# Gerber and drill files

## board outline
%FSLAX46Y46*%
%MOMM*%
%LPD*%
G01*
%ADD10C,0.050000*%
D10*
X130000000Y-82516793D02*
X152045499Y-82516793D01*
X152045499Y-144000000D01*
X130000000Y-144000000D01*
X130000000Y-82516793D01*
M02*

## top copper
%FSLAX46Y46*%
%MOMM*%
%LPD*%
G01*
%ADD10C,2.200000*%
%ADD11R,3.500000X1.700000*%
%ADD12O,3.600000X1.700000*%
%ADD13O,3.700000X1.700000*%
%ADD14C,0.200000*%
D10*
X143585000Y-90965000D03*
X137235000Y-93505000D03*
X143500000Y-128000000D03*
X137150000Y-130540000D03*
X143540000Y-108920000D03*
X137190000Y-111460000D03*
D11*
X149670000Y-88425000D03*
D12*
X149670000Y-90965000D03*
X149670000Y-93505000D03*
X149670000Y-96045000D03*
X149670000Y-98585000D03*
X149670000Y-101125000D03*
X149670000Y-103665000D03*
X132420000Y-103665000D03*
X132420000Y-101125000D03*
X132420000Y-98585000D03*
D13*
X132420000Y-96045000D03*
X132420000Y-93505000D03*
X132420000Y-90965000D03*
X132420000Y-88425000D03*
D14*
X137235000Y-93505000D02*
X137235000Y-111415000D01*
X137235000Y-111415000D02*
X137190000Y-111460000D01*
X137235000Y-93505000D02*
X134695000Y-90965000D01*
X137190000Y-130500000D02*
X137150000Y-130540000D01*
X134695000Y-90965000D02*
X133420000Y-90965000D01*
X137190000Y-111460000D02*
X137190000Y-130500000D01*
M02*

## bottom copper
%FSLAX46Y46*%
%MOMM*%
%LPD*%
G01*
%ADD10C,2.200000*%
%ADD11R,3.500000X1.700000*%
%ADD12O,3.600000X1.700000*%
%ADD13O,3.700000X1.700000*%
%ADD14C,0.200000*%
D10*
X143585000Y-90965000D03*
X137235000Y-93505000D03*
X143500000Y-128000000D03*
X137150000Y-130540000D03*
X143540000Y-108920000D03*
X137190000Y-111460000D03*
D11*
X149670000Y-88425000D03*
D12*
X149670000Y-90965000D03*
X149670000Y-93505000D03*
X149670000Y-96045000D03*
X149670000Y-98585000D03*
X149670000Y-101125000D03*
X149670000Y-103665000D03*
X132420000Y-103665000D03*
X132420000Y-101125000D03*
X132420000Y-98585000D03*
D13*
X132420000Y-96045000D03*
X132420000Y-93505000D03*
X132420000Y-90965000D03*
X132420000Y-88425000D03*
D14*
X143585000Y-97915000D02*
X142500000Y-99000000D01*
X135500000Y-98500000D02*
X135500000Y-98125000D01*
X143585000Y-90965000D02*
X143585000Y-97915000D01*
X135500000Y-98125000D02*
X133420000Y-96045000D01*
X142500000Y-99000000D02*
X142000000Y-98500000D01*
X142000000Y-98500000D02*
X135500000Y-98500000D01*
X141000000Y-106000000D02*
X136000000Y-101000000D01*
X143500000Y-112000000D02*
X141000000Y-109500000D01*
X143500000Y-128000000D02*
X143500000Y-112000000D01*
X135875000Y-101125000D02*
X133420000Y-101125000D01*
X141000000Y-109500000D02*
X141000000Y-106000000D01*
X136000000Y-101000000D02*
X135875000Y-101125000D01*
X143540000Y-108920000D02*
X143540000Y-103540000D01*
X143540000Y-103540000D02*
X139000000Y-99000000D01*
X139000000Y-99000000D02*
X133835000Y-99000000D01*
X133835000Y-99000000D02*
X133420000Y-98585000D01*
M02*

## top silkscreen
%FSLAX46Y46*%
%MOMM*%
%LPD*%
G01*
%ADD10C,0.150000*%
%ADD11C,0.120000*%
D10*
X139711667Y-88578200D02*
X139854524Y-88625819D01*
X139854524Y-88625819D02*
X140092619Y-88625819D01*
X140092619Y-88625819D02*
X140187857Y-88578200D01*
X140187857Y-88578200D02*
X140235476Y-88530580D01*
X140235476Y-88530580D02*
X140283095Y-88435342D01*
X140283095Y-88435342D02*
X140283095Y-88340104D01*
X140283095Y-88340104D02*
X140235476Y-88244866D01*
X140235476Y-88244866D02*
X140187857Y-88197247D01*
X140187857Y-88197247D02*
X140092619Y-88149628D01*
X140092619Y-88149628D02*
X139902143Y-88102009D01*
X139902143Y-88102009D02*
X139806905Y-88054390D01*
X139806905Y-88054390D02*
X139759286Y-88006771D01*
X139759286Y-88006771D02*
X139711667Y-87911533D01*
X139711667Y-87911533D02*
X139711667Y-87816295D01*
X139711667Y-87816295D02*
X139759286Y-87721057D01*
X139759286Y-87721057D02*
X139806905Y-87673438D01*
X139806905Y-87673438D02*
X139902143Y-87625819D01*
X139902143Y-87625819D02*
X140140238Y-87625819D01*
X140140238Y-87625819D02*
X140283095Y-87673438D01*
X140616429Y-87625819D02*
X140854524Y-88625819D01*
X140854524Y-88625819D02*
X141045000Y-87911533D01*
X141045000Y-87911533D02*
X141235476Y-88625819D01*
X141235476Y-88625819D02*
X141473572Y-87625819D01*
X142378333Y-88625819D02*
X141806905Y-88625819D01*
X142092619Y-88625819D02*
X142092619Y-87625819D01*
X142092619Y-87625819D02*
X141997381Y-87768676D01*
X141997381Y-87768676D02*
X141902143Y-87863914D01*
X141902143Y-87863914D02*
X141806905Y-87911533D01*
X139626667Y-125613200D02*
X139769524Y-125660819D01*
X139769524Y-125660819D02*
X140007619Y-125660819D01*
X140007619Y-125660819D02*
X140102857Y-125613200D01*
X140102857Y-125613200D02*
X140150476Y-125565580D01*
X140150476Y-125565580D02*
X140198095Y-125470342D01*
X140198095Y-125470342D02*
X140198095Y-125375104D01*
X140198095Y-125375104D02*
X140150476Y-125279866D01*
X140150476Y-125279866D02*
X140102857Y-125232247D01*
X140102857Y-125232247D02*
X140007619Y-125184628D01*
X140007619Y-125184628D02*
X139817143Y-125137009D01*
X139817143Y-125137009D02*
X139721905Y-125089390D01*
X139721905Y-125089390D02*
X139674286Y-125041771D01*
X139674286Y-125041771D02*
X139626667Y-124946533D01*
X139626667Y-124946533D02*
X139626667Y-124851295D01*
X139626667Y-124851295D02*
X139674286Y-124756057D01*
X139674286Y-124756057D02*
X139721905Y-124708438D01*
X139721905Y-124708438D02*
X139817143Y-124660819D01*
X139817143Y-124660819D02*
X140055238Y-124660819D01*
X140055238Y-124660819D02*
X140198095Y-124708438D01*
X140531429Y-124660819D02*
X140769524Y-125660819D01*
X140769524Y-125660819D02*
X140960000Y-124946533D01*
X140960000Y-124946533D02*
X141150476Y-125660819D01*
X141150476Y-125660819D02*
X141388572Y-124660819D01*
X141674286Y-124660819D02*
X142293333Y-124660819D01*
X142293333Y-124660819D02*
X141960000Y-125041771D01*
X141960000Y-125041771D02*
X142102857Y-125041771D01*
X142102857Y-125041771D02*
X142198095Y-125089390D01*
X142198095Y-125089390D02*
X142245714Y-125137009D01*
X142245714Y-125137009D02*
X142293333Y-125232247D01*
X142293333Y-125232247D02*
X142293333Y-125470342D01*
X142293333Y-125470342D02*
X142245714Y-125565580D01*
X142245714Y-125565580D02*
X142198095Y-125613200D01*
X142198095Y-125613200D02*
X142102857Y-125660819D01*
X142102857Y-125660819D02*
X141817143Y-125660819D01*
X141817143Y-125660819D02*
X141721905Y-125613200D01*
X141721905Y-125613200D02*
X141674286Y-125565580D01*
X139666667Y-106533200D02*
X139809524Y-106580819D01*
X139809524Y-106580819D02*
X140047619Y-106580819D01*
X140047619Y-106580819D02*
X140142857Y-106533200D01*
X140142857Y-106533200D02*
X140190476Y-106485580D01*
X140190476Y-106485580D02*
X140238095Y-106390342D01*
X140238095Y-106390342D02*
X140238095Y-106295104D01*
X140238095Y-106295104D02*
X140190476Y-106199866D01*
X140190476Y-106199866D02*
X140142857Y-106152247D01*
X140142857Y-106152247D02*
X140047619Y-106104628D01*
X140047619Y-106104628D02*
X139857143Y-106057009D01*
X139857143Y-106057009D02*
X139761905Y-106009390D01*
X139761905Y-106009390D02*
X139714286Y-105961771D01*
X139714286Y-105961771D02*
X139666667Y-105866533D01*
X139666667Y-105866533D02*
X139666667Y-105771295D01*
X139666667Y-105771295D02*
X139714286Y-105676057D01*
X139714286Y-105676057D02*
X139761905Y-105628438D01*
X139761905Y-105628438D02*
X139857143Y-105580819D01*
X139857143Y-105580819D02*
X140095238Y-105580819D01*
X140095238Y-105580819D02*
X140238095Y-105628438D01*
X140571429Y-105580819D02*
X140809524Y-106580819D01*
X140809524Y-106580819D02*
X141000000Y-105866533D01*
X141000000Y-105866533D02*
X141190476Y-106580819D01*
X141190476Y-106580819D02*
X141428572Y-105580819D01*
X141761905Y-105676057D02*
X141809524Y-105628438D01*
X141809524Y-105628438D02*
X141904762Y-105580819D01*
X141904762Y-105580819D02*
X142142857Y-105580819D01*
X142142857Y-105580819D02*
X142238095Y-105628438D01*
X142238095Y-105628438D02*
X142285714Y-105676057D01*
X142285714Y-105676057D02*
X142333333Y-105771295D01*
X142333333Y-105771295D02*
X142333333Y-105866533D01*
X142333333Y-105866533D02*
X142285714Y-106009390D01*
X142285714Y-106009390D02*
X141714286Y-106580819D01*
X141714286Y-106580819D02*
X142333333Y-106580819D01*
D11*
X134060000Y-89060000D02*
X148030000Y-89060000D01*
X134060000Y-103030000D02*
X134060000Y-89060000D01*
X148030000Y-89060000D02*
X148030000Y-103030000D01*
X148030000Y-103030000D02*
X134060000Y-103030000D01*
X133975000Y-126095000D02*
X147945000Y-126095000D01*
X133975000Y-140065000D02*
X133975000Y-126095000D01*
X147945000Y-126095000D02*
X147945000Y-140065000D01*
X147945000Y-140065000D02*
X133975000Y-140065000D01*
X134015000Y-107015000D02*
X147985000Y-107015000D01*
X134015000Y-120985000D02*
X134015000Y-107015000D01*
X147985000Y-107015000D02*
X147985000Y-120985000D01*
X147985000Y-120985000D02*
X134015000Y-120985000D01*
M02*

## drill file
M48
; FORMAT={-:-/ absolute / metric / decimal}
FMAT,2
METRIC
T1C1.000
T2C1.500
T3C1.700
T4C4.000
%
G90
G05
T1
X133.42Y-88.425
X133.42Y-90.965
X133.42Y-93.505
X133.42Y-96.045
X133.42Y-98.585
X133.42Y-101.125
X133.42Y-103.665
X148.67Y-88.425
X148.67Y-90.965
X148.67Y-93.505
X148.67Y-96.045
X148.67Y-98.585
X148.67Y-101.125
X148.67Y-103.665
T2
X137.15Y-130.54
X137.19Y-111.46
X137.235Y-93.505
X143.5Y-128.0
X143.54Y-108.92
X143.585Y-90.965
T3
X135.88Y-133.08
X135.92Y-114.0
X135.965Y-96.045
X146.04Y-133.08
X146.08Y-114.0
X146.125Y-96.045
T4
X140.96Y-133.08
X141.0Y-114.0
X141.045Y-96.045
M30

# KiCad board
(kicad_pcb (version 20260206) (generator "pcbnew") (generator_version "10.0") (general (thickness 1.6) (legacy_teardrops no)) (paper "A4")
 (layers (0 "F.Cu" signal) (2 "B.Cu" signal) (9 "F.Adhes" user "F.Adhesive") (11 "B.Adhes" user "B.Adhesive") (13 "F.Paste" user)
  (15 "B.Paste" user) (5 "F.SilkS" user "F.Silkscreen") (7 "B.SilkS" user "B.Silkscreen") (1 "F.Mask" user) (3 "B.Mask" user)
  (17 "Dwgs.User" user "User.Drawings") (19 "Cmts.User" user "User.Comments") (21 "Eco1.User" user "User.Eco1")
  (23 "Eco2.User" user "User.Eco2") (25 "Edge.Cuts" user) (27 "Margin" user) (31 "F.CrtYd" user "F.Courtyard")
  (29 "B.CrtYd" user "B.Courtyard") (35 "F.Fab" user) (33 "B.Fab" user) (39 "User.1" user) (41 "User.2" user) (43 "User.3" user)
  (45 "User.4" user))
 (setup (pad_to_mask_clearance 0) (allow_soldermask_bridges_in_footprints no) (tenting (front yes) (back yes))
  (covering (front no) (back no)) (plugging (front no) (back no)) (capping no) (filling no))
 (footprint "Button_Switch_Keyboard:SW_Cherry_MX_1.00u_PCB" (layer "F.Cu") (at 143.585 90.965)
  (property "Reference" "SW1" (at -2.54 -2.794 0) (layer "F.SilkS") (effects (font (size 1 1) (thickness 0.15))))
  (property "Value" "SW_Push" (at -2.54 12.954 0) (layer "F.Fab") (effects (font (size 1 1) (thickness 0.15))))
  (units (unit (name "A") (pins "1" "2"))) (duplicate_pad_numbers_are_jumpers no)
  (fp_line (start -9.525 -1.905) (end 4.445 -1.905) (stroke (width 0.12) (type solid)) (layer "F.SilkS"))
  (fp_line (start -9.525 12.065) (end -9.525 -1.905) (stroke (width 0.12) (type solid)) (layer "F.SilkS"))
  (fp_line (start 4.445 -1.905) (end 4.445 12.065) (stroke (width 0.12) (type solid)) (layer "F.SilkS"))
  (fp_line (start 4.445 12.065) (end -9.525 12.065) (stroke (width 0.12) (type solid)) (layer "F.SilkS"))
  (pad "" np_thru_hole circle (at -7.62 5.08) (size 1.7 1.7) (drill 1.7) (layers "*.Cu" "*.Mask"))
  (pad "" np_thru_hole circle (at -2.54 5.08) (size 4 4) (drill 4) (layers "*.Cu" "*.Mask"))
  (pad "" np_thru_hole circle (at 2.54 5.08) (size 1.7 1.7) (drill 1.7) (layers "*.Cu" "*.Mask"))
  (pad "1" thru_hole circle (at 0 0) (size 2.2 2.2) (drill 1.5) (layers "*.Cu" "*.Mask") (remove_unused_layers no)
   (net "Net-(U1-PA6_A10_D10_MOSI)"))
  (pad "2" thru_hole circle (at -6.35 2.54) (size 2.2 2.2) (drill 1.5) (layers "*.Cu" "*.Mask") (remove_unused_layers no) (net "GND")))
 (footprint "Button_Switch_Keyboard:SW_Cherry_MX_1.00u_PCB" (layer "F.Cu") (at 143.5 128)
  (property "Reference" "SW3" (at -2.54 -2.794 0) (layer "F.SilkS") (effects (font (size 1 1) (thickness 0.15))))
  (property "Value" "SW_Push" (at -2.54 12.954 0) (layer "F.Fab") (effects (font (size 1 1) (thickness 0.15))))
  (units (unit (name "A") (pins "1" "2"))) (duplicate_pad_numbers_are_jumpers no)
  (fp_line (start -9.525 -1.905) (end 4.445 -1.905) (stroke (width 0.12) (type solid)) (layer "F.SilkS"))
  (fp_line (start -9.525 12.065) (end -9.525 -1.905) (stroke (width 0.12) (type solid)) (layer "F.SilkS"))
  (fp_line (start 4.445 -1.905) (end 4.445 12.065) (stroke (width 0.12) (type solid)) (layer "F.SilkS"))
  (fp_line (start 4.445 12.065) (end -9.525 12.065) (stroke (width 0.12) (type solid)) (layer "F.SilkS"))
  (pad "" np_thru_hole circle (at -7.62 5.08) (size 1.7 1.7) (drill 1.7) (layers "*.Cu" "*.Mask"))
  (pad "" np_thru_hole circle (at -2.54 5.08) (size 4 4) (drill 4) (layers "*.Cu" "*.Mask"))
  (pad "" np_thru_hole circle (at 2.54 5.08) (size 1.7 1.7) (drill 1.7) (layers "*.Cu" "*.Mask"))
  (pad "1" thru_hole circle (at 0 0) (size 2.2 2.2) (drill 1.5) (layers "*.Cu" "*.Mask") (remove_unused_layers no)
   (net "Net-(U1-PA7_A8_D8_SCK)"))
  (pad "2" thru_hole circle (at -6.35 2.54) (size 2.2 2.2) (drill 1.5) (layers "*.Cu" "*.Mask") (remove_unused_layers no) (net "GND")))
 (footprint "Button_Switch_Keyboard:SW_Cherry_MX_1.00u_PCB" (layer "F.Cu") (at 143.54 108.92)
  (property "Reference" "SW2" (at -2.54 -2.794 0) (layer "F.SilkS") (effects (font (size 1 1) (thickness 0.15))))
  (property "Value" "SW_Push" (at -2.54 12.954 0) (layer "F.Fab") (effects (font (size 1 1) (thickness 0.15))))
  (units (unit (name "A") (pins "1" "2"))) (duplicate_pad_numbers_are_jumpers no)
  (fp_line (start -9.525 -1.905) (end 4.445 -1.905) (stroke (width 0.12) (type solid)) (layer "F.SilkS"))
  (fp_line (start -9.525 12.065) (end -9.525 -1.905) (stroke (width 0.12) (type solid)) (layer "F.SilkS"))
  (fp_line (start 4.445 -1.905) (end 4.445 12.065) (stroke (width 0.12) (type solid)) (layer "F.SilkS"))
  (fp_line (start 4.445 12.065) (end -9.525 12.065) (stroke (width 0.12) (type solid)) (layer "F.SilkS"))
  (pad "" np_thru_hole circle (at -7.62 5.08) (size 1.7 1.7) (drill 1.7) (layers "*.Cu" "*.Mask"))
  (pad "" np_thru_hole circle (at -2.54 5.08) (size 4 4) (drill 4) (layers "*.Cu" "*.Mask"))
  (pad "" np_thru_hole circle (at 2.54 5.08) (size 1.7 1.7) (drill 1.7) (layers "*.Cu" "*.Mask"))
  (pad "1" thru_hole circle (at 0 0) (size 2.2 2.2) (drill 1.5) (layers "*.Cu" "*.Mask") (remove_unused_layers no)
   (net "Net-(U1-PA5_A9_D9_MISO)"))
  (pad "2" thru_hole circle (at -6.35 2.54) (size 2.2 2.2) (drill 1.5) (layers "*.Cu" "*.Mask") (remove_unused_layers no) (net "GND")))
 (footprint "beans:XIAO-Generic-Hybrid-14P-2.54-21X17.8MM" (layer "B.Cu") (at 141.045 96.045 180)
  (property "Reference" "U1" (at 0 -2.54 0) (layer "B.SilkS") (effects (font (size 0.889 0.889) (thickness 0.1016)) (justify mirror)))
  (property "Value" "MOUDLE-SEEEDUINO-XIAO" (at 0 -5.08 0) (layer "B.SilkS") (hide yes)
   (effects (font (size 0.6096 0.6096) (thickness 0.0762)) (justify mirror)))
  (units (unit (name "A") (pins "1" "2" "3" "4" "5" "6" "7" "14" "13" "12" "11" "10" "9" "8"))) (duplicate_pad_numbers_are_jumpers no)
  (pad "1" thru_hole rect (at -7.625 7.62 180) (size 3.5 1.7) (drill 1 (offset -1 0)) (layers "*.Cu" "*.Mask") (remove_unused_layers no)
   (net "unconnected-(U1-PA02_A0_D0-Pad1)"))
  (pad "2" thru_hole oval (at -7.625 5.08 180) (size 3.6 1.7) (drill 1 (offset -1 0)) (layers "*.Cu" "*.Mask") (remove_unused_layers no)
   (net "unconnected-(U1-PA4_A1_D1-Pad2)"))
  (pad "3" thru_hole oval (at -7.625 2.54 180) (size 3.6 1.7) (drill 1 (offset -1 0)) (layers "*.Cu" "*.Mask") (remove_unused_layers no)
   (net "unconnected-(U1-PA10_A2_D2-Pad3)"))
  (pad "4" thru_hole oval (at -7.625 0 180) (size 3.6 1.7) (drill 1 (offset -1 0)) (layers "*.Cu" "*.Mask") (remove_unused_layers no)
   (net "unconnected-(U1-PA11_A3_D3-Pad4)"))
  (pad "5" thru_hole oval (at -7.625 -2.54 180) (size 3.6 1.7) (drill 1 (offset -1 0)) (layers "*.Cu" "*.Mask") (remove_unused_layers no)
   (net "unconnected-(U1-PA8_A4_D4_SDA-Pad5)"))
  (pad "6" thru_hole oval (at -7.625 -5.08) (size 3.6 1.7) (drill 1 (offset 1 0)) (layers "*.Cu" "*.Mask") (remove_unused_layers no)
   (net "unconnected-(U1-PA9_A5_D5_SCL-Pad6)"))
  (pad "7" thru_hole oval (at -7.625 -7.62 180) (size 3.6 1.7) (drill 1 (offset -1 0)) (layers "*.Cu" "*.Mask") (remove_unused_layers no)
   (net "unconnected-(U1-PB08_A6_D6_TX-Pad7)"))
  (pad "8" thru_hole oval (at 7.625 -7.62 180) (size 3.6 1.7) (drill 1 (offset 1 0)) (layers "*.Cu" "*.Mask") (remove_unused_layers no)
   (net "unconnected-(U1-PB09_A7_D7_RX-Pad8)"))
  (pad "9" thru_hole oval (at 7.625 -5.08 180) (size 3.6 1.7) (drill 1 (offset 1 0)) (layers "*.Cu" "*.Mask") (remove_unused_layers no)
   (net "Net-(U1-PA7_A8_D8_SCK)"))
  (pad "10" thru_hole oval (at 7.625 -2.54 180) (size 3.6 1.7) (drill 1 (offset 1 0)) (layers "*.Cu" "*.Mask") (remove_unused_layers no)
   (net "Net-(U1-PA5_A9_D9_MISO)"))
  (pad "11" thru_hole oval (at 7.625 0 180) (size 3.7 1.7) (drill 1 (offset 1 0)) (layers "*.Cu" "*.Mask") (remove_unused_layers no)
   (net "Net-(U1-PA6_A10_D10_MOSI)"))
  (pad "12" thru_hole oval (at 7.625 2.54 180) (size 3.7 1.7) (drill 1 (offset 1 0)) (layers "*.Cu" "*.Mask") (remove_unused_layers no)
   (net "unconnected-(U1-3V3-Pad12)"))
  (pad "13" thru_hole oval (at 7.625 5.08 180) (size 3.7 1.7) (drill 1 (offset 1 0)) (layers "*.Cu" "*.Mask") (remove_unused_layers no)
   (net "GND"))
  (pad "14" thru_hole oval (at 7.625 7.62 180) (size 3.7 1.7) (drill 1 (offset 1 0)) (layers "*.Cu" "*.Mask") (remove_unused_layers no)
   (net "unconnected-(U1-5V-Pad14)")))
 (gr_rect (start 130 82.516793) (end 152.045499 144) (stroke (width 0.05) (type default)) (fill no) (layer "Edge.Cuts"))
 (segment (start 143.585 97.915) (end 142.5 99) (width 0.2) (layer "B.Cu") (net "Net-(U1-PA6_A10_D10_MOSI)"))
 (segment (start 135.5 98.5) (end 135.5 98.125) (width 0.2) (layer "B.Cu") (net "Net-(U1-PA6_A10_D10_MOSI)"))
 (segment (start 143.585 90.965) (end 143.585 97.915) (width 0.2) (layer "B.Cu") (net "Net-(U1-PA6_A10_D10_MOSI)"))
 (segment (start 135.5 98.125) (end 133.42 96.045) (width 0.2) (layer "B.Cu") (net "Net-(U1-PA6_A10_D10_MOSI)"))
 (segment (start 142.5 99) (end 142 98.5) (width 0.2) (layer "B.Cu") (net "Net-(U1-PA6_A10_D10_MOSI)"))
 (segment (start 142 98.5) (end 135.5 98.5) (width 0.2) (layer "B.Cu") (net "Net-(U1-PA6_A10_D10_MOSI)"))
 (segment (start 137.235 93.505) (end 137.235 111.415) (width 0.2) (layer "F.Cu") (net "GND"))
 (segment (start 137.235 111.415) (end 137.19 111.46) (width 0.2) (layer "F.Cu") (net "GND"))
 (segment (start 137.235 93.505) (end 134.695 90.965) (width 0.2) (layer "F.Cu") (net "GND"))
 (segment (start 137.19 130.5) (end 137.15 130.54) (width 0.2) (layer "F.Cu") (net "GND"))
 (segment (start 134.695 90.965) (end 133.42 90.965) (width 0.2) (layer "F.Cu") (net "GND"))
 (segment (start 137.19 111.46) (end 137.19 130.5) (width 0.2) (layer "F.Cu") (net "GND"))
 (segment (start 141 106) (end 136 101) (width 0.2) (layer "B.Cu") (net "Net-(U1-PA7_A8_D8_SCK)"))
 (segment (start 143.5 112) (end 141 109.5) (width 0.2) (layer "B.Cu") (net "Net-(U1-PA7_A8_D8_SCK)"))
 (segment (start 143.5 128) (end 143.5 112) (width 0.2) (layer "B.Cu") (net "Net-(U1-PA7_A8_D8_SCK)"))
 (segment (start 135.875 101.125) (end 133.42 101.125) (width 0.2) (layer "B.Cu") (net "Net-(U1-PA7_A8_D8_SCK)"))
 (segment (start 141 109.5) (end 141 106) (width 0.2) (layer "B.Cu") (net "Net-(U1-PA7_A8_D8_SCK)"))
 (segment (start 136 101) (end 135.875 101.125) (width 0.2) (layer "B.Cu") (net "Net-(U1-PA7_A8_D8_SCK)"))
 (segment (start 143.54 108.92) (end 143.54 103.54) (width 0.2) (layer "B.Cu") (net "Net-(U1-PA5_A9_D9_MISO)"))
 (segment (start 143.54 103.54) (end 139 99) (width 0.2) (layer "B.Cu") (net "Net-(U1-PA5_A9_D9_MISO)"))
 (segment (start 139 99) (end 133.835 99) (width 0.2) (layer "B.Cu") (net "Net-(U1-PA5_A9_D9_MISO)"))
 (segment (start 133.835 99) (end 133.42 98.585) (width 0.2) (layer "B.Cu") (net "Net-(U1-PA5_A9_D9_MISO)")))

